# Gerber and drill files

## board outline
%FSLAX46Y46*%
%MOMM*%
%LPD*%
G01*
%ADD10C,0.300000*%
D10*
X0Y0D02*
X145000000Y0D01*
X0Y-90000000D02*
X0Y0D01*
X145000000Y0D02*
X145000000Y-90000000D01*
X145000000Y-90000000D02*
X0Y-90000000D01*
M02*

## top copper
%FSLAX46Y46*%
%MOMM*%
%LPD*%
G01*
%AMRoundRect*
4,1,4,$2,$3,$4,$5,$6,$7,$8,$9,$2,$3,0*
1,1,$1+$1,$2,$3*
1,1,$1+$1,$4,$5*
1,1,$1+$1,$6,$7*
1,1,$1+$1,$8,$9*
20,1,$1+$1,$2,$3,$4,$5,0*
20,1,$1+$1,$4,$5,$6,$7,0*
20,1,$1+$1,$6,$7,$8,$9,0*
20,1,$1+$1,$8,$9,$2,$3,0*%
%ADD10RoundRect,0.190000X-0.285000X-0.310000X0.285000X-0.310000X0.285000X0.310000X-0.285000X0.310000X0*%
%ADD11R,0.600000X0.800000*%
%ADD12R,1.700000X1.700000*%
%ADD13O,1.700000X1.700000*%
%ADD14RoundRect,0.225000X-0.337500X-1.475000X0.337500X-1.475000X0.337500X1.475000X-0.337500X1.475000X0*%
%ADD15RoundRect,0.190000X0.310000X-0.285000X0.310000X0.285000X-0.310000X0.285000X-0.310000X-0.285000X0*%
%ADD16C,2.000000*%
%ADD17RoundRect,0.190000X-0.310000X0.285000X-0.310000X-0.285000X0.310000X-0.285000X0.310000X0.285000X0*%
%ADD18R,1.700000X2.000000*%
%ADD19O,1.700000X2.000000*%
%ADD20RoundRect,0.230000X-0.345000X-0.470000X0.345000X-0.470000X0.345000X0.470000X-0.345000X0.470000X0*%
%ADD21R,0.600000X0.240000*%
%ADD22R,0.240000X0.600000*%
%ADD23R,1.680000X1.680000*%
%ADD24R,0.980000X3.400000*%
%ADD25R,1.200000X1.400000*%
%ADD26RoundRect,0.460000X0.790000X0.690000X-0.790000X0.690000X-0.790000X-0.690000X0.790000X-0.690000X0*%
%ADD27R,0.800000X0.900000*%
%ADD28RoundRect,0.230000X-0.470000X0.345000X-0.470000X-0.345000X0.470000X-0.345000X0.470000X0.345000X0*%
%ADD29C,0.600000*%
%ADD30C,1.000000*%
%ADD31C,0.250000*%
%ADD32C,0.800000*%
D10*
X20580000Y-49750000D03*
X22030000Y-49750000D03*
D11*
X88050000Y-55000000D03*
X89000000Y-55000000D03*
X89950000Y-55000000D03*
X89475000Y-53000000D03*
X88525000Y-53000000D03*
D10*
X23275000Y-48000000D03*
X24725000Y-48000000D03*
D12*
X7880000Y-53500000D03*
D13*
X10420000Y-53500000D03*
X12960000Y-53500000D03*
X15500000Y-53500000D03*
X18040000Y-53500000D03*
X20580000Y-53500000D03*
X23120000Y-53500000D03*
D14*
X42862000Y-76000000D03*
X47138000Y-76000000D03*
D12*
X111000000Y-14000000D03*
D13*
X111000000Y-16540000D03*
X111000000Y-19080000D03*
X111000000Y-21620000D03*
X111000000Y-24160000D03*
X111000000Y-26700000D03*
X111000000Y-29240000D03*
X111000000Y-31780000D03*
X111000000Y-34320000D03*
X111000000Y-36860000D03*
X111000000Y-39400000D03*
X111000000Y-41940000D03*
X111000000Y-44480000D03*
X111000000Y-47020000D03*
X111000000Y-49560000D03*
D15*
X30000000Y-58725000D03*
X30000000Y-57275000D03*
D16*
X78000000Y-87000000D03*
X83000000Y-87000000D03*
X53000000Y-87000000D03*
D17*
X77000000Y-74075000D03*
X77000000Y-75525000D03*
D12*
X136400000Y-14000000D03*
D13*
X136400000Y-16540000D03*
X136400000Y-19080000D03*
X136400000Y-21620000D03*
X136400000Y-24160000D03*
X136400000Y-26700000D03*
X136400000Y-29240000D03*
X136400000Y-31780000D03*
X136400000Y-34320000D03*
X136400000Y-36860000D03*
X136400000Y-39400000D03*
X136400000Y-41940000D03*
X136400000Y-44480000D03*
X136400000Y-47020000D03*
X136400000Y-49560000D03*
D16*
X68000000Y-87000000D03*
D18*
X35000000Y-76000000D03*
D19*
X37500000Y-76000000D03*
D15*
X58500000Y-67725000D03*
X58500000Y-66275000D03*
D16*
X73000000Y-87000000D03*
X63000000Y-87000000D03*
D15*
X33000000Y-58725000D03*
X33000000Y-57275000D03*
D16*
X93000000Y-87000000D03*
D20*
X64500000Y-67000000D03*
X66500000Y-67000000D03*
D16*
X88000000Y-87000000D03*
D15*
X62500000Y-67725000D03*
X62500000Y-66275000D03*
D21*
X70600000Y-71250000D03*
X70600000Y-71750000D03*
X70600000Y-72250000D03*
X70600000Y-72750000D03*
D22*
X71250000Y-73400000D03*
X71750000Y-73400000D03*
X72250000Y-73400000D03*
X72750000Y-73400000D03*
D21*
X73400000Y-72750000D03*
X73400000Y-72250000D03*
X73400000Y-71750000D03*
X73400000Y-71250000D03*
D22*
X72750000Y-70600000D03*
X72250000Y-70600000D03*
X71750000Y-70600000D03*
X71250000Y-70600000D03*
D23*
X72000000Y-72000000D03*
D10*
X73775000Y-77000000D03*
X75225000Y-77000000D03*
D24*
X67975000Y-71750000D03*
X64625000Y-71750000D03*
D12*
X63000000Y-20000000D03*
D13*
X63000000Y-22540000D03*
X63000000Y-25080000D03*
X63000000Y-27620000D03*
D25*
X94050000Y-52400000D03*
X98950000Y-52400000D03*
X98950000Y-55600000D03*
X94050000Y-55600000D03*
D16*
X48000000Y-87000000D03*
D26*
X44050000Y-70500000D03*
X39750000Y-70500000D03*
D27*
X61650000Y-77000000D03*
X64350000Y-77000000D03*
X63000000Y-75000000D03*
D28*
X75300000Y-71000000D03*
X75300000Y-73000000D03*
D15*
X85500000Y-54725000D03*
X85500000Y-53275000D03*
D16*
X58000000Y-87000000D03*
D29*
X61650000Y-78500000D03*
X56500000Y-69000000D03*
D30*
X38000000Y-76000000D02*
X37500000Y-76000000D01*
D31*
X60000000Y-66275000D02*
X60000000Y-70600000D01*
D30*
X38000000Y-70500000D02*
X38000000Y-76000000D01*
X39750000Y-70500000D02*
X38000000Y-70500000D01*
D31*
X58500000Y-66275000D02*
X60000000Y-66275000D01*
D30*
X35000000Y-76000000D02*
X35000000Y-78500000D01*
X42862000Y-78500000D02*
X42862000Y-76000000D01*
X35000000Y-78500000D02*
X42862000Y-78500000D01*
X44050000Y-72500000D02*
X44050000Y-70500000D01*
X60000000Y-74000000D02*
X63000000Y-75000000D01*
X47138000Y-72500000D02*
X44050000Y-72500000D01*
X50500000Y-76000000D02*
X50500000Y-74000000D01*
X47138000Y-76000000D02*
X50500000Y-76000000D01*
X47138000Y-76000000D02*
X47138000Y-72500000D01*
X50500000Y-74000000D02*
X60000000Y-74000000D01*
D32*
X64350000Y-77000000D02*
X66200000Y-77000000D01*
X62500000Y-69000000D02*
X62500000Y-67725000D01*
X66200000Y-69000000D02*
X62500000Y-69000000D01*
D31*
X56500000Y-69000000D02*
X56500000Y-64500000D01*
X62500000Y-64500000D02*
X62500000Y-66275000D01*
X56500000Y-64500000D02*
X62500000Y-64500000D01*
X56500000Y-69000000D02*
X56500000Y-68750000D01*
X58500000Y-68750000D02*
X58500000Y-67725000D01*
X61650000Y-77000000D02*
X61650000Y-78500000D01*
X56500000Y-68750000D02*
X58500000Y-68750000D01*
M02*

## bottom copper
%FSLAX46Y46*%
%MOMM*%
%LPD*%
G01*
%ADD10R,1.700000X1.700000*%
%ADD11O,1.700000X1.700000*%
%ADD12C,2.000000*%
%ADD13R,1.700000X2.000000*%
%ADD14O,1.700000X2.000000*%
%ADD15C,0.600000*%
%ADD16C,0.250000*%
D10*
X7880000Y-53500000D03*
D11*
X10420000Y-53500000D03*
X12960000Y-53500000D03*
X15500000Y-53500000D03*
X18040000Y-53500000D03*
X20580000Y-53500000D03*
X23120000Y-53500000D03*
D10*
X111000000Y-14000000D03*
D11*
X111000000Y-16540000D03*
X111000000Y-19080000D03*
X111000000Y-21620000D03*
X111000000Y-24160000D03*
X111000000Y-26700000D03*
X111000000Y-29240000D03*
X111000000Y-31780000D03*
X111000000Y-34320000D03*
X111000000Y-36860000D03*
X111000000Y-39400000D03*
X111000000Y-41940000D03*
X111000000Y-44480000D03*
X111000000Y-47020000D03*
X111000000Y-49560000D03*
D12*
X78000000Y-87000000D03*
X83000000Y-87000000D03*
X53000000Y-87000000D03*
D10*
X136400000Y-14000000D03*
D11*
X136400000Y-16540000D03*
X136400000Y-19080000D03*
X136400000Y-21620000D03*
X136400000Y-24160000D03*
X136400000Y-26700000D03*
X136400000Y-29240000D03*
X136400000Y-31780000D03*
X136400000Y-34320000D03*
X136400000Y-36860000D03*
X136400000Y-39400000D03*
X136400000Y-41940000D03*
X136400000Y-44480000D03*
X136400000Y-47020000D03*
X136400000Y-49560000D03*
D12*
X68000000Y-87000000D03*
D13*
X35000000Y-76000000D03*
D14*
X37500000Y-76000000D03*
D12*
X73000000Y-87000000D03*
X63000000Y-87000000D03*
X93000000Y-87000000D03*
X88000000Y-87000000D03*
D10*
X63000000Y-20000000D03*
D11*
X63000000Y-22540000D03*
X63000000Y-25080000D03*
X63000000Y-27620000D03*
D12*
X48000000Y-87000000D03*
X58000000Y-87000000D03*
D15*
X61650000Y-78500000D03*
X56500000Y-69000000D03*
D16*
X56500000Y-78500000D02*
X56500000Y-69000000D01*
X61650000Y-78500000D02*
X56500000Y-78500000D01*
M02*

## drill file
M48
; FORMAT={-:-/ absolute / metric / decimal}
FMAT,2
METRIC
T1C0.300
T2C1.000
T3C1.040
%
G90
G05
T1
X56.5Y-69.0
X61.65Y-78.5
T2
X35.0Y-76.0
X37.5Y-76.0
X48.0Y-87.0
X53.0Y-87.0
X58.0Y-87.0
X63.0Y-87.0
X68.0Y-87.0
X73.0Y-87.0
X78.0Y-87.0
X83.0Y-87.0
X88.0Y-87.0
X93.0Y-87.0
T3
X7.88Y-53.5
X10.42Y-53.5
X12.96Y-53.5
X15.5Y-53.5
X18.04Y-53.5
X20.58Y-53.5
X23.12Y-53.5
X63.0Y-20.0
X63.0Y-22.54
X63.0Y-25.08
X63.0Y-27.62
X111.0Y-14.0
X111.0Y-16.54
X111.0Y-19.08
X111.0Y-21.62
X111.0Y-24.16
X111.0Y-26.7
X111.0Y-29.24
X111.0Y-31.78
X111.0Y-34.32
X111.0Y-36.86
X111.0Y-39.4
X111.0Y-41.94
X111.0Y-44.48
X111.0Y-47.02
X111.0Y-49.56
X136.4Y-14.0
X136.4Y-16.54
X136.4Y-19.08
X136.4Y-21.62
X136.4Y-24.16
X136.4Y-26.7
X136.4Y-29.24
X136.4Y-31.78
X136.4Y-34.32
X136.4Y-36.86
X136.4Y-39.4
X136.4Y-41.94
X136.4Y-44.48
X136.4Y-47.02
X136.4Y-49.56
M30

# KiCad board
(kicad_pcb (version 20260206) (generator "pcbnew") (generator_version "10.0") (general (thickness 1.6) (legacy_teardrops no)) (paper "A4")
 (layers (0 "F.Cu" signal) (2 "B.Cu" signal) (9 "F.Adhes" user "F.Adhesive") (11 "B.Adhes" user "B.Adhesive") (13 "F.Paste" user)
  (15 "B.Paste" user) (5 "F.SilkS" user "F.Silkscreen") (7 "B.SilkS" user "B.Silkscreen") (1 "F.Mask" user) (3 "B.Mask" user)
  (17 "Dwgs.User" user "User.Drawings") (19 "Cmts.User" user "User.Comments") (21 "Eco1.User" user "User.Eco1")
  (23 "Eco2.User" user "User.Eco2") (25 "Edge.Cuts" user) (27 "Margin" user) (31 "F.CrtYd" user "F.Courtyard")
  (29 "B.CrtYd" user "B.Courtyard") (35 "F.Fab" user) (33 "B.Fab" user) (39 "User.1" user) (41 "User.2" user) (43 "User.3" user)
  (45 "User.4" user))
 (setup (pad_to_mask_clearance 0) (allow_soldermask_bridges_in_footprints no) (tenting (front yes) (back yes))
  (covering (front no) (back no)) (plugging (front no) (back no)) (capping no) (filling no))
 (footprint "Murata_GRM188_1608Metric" (layer "F.Cu") (at 21.305 49.75)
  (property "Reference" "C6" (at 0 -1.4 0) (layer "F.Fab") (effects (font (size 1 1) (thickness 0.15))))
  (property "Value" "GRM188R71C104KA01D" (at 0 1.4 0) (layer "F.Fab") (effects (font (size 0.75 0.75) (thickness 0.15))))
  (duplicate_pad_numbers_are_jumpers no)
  (pad "1" smd roundrect (at -0.725 0) (size 0.95 1) (layers "F.Cu" "F.Mask" "F.Paste") (roundrect_rratio 0.2) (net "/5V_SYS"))
  (pad "2" smd roundrect (at 0.725 0) (size 0.95 1) (layers "F.Cu" "F.Mask" "F.Paste") (roundrect_rratio 0.2) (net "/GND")))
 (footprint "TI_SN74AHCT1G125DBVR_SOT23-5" (layer "F.Cu") (at 89 54)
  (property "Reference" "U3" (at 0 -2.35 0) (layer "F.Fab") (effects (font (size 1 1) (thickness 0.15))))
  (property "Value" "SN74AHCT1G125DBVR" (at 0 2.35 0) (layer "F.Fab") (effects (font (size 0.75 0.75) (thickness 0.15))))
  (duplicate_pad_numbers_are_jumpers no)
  (pad "1" smd rect (at -0.95 1) (size 0.6 0.8) (layers "F.Cu" "F.Mask" "F.Paste") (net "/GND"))
  (pad "2" smd rect (at 0 1) (size 0.6 0.8) (layers "F.Cu" "F.Mask" "F.Paste") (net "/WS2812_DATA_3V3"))
  (pad "3" smd rect (at 0.95 1) (size 0.6 0.8) (layers "F.Cu" "F.Mask" "F.Paste") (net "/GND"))
  (pad "4" smd rect (at 0.475 -1) (size 0.6 0.8) (layers "F.Cu" "F.Mask" "F.Paste") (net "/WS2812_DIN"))
  (pad "5" smd rect (at -0.475 -1) (size 0.6 0.8) (layers "F.Cu" "F.Mask" "F.Paste") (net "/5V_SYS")))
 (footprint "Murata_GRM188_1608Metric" (layer "F.Cu") (at 24 48)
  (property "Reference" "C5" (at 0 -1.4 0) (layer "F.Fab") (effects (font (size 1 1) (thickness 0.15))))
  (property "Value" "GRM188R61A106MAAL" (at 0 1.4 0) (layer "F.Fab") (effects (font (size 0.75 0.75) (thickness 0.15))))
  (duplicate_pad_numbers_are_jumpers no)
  (pad "1" smd roundrect (at -0.725 0) (size 0.95 1) (layers "F.Cu" "F.Mask" "F.Paste") (roundrect_rratio 0.2) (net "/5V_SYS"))
  (pad "2" smd roundrect (at 0.725 0) (size 0.95 1) (layers "F.Cu" "F.Mask" "F.Paste") (roundrect_rratio 0.2) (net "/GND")))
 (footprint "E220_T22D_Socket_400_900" (layer "F.Cu") (at 5 52)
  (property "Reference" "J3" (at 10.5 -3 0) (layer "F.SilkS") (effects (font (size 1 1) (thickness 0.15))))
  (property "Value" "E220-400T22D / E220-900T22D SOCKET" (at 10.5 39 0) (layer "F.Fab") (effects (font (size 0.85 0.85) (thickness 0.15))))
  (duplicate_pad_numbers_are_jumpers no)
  (pad "1" thru_hole rect (at 2.88 1.5) (size 1.7 1.7) (drill 1.04) (layers "*.Cu" "*.Mask") (remove_unused_layers no) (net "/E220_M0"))
  (pad "2" thru_hole oval (at 5.42 1.5) (size 1.7 1.7) (drill 1.04) (layers "*.Cu" "*.Mask") (remove_unused_layers no) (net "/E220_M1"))
  (pad "3" thru_hole oval (at 7.96 1.5) (size 1.7 1.7) (drill 1.04) (layers "*.Cu" "*.Mask") (remove_unused_layers no) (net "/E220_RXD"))
  (pad "4" thru_hole oval (at 10.5 1.5) (size 1.7 1.7) (drill 1.04) (layers "*.Cu" "*.Mask") (remove_unused_layers no) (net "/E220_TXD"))
  (pad "5" thru_hole oval (at 13.04 1.5) (size 1.7 1.7) (drill 1.04) (layers "*.Cu" "*.Mask") (remove_unused_layers no) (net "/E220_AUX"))
  (pad "6" thru_hole oval (at 15.58 1.5) (size 1.7 1.7) (drill 1.04) (layers "*.Cu" "*.Mask") (remove_unused_layers no) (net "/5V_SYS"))
  (pad "7" thru_hole oval (at 18.12 1.5) (size 1.7 1.7) (drill 1.04) (layers "*.Cu" "*.Mask") (remove_unused_layers no) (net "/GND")))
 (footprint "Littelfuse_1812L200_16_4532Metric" (layer "F.Cu") (at 45 76)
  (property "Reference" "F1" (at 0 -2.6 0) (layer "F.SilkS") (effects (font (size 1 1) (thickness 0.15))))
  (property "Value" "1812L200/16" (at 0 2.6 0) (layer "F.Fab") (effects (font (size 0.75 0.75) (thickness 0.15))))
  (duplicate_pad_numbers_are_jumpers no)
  (pad "1" smd roundrect (at -2.138 0) (size 1.125 3.4) (layers "F.Cu" "F.Mask" "F.Paste") (roundrect_rratio 0.2) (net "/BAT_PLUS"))
  (pad "2" smd roundrect (at 2.138 0) (size 1.125 3.4) (layers "F.Cu" "F.Mask" "F.Paste") (roundrect_rratio 0.2) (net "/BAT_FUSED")))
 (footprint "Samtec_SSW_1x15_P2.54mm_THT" (layer "F.Cu") (at 111 14)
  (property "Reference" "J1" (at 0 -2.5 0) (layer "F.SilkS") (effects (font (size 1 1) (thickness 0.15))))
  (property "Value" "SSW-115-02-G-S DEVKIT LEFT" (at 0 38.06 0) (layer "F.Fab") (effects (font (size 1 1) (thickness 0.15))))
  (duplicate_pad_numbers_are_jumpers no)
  (pad "1" thru_hole rect (at 0 0) (size 1.7 1.7) (drill 1.04) (layers "*.Cu" "*.Mask") (remove_unused_layers no) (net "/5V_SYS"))
  (pad "2" thru_hole oval (at 0 2.54) (size 1.7 1.7) (drill 1.04) (layers "*.Cu" "*.Mask") (remove_unused_layers no) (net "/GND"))
  (pad "3" thru_hole oval (at 0 5.08) (size 1.7 1.7) (drill 1.04) (layers "*.Cu" "*.Mask") (remove_unused_layers no))
  (pad "4" thru_hole oval (at 0 7.62) (size 1.7 1.7) (drill 1.04) (layers "*.Cu" "*.Mask") (remove_unused_layers no))
  (pad "5" thru_hole oval (at 0 10.16) (size 1.7 1.7) (drill 1.04) (layers "*.Cu" "*.Mask") (remove_unused_layers no))
  (pad "6" thru_hole oval (at 0 12.7) (size 1.7 1.7) (drill 1.04) (layers "*.Cu" "*.Mask") (remove_unused_layers no) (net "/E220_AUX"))
  (pad "7" thru_hole oval (at 0 15.24) (size 1.7 1.7) (drill 1.04) (layers "*.Cu" "*.Mask") (remove_unused_layers no) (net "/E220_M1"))
  (pad "8" thru_hole oval (at 0 17.78) (size 1.7 1.7) (drill 1.04) (layers "*.Cu" "*.Mask") (remove_unused_layers no) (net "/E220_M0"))
  (pad "9" thru_hole oval (at 0 20.32) (size 1.7 1.7) (drill 1.04) (layers "*.Cu" "*.Mask") (remove_unused_layers no))
  (pad "10" thru_hole oval (at 0 22.86) (size 1.7 1.7) (drill 1.04) (layers "*.Cu" "*.Mask") (remove_unused_layers no))
  (pad "11" thru_hole oval (at 0 25.4) (size 1.7 1.7) (drill 1.04) (layers "*.Cu" "*.Mask") (remove_unused_layers no))
  (pad "12" thru_hole oval (at 0 27.94) (size 1.7 1.7) (drill 1.04) (layers "*.Cu" "*.Mask") (remove_unused_layers no))
  (pad "13" thru_hole oval (at 0 30.48) (size 1.7 1.7) (drill 1.04) (layers "*.Cu" "*.Mask") (remove_unused_layers no))
  (pad "14" thru_hole oval (at 0 33.02) (size 1.7 1.7) (drill 1.04) (layers "*.Cu" "*.Mask") (remove_unused_layers no))
  (pad "15" thru_hole oval (at 0 35.56) (size 1.7 1.7) (drill 1.04) (layers "*.Cu" "*.Mask") (remove_unused_layers no)))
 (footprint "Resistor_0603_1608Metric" (layer "F.Cu") (at 30 58 90)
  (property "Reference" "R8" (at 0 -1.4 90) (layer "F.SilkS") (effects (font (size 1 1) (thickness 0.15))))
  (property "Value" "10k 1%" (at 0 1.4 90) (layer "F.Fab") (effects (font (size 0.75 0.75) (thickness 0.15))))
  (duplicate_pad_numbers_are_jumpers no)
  (pad "1" smd roundrect (at -0.725 0 90) (size 0.95 1) (layers "F.Cu" "F.Mask" "F.Paste") (roundrect_rratio 0.2) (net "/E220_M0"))
  (pad "2" smd roundrect (at 0.725 0 90) (size 0.95 1) (layers "F.Cu" "F.Mask" "F.Paste") (roundrect_rratio 0.2) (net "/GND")))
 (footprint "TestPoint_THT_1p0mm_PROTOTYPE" (layer "F.Cu") (at 78 87)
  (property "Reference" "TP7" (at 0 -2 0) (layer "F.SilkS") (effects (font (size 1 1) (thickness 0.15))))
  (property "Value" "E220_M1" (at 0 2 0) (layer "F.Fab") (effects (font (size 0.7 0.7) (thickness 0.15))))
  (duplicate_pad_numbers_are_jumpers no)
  (pad "1" thru_hole circle (at 0 0) (size 2 2) (drill 1) (layers "*.Cu" "*.Mask") (remove_unused_layers no) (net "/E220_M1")))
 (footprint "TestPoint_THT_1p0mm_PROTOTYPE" (layer "F.Cu") (at 83 87)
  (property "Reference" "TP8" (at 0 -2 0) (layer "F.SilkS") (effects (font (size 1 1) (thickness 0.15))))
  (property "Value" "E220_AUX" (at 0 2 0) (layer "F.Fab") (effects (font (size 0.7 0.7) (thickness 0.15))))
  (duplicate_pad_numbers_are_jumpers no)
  (pad "1" thru_hole circle (at 0 0) (size 2 2) (drill 1) (layers "*.Cu" "*.Mask") (remove_unused_layers no) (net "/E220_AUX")))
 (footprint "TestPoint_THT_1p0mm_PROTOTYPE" (layer "F.Cu") (at 53 87)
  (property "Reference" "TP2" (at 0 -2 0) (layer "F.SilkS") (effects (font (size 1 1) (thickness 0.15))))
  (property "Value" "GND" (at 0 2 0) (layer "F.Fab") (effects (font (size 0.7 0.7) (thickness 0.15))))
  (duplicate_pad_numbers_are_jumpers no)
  (pad "1" thru_hole circle (at 0 0) (size 2 2) (drill 1) (layers "*.Cu" "*.Mask") (remove_unused_layers no) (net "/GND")))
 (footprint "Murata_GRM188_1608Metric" (layer "F.Cu") (at 77 74.8 -90)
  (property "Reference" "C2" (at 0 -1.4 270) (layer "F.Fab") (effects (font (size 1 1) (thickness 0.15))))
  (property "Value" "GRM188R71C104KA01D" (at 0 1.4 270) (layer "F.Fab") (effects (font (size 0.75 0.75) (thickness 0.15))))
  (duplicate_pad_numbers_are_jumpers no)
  (pad "1" smd roundrect (at -0.725 0 270) (size 0.95 1) (layers "F.Cu" "F.Mask" "F.Paste") (roundrect_rratio 0.2) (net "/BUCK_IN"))
  (pad "2" smd roundrect (at 0.725 0 270) (size 0.95 1) (layers "F.Cu" "F.Mask" "F.Paste") (roundrect_rratio 0.2) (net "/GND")))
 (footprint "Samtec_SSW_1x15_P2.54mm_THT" (layer "F.Cu") (at 136.4 14)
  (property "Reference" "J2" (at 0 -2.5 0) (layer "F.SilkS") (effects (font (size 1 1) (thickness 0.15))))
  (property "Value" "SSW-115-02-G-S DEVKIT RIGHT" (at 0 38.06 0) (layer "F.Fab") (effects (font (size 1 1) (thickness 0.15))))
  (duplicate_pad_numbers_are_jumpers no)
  (pad "1" thru_hole rect (at 0 0) (size 1.7 1.7) (drill 1.04) (layers "*.Cu" "*.Mask") (remove_unused_layers no) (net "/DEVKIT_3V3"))
  (pad "2" thru_hole oval (at 0 2.54) (size 1.7 1.7) (drill 1.04) (layers "*.Cu" "*.Mask") (remove_unused_layers no) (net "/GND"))
  (pad "3" thru_hole oval (at 0 5.08) (size 1.7 1.7) (drill 1.04) (layers "*.Cu" "*.Mask") (remove_unused_layers no))
  (pad "4" thru_hole oval (at 0 7.62) (size 1.7 1.7) (drill 1.04) (layers "*.Cu" "*.Mask") (remove_unused_layers no))
  (pad "5" thru_hole oval (at 0 10.16) (size 1.7 1.7) (drill 1.04) (layers "*.Cu" "*.Mask") (remove_unused_layers no)
   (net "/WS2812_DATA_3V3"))
  (pad "6" thru_hole oval (at 0 12.7) (size 1.7 1.7) (drill 1.04) (layers "*.Cu" "*.Mask") (remove_unused_layers no) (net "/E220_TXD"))
  (pad "7" thru_hole oval (at 0 15.24) (size 1.7 1.7) (drill 1.04) (layers "*.Cu" "*.Mask") (remove_unused_layers no) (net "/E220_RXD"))
  (pad "8" thru_hole oval (at 0 17.78) (size 1.7 1.7) (drill 1.04) (layers "*.Cu" "*.Mask") (remove_unused_layers no))
  (pad "9" thru_hole oval (at 0 20.32) (size 1.7 1.7) (drill 1.04) (layers "*.Cu" "*.Mask") (remove_unused_layers no))
  (pad "10" thru_hole oval (at 0 22.86) (size 1.7 1.7) (drill 1.04) (layers "*.Cu" "*.Mask") (remove_unused_layers no))
  (pad "11" thru_hole oval (at 0 25.4) (size 1.7 1.7) (drill 1.04) (layers "*.Cu" "*.Mask") (remove_unused_layers no) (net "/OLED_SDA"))
  (pad "12" thru_hole oval (at 0 27.94) (size 1.7 1.7) (drill 1.04) (layers "*.Cu" "*.Mask") (remove_unused_layers no))
  (pad "13" thru_hole oval (at 0 30.48) (size 1.7 1.7) (drill 1.04) (layers "*.Cu" "*.Mask") (remove_unused_layers no))
  (pad "14" thru_hole oval (at 0 33.02) (size 1.7 1.7) (drill 1.04) (layers "*.Cu" "*.Mask") (remove_unused_layers no) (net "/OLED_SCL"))
  (pad "15" thru_hole oval (at 0 35.56) (size 1.7 1.7) (drill 1.04) (layers "*.Cu" "*.Mask") (remove_unused_layers no)))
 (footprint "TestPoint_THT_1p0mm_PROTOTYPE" (layer "F.Cu") (at 68 87)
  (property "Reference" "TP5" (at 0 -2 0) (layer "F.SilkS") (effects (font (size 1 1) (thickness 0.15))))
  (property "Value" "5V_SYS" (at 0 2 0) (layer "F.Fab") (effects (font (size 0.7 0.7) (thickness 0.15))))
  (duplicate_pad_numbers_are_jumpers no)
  (pad "1" thru_hole circle (at 0 0) (size 2 2) (drill 1) (layers "*.Cu" "*.Mask") (remove_unused_layers no) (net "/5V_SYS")))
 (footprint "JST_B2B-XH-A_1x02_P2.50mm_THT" (layer "F.Cu") (at 35 76)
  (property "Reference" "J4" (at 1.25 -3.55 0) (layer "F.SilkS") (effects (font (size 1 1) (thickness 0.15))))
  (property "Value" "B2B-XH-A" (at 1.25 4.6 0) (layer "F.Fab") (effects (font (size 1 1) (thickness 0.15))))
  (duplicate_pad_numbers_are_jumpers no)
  (pad "1" thru_hole rect (at 0 0) (size 1.7 2) (drill 1) (layers "*.Cu" "*.Mask") (remove_unused_layers no) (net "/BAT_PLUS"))
  (pad "2" thru_hole oval (at 2.5 0) (size 1.7 2) (drill 1) (layers "*.Cu" "*.Mask") (remove_unused_layers no) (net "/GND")))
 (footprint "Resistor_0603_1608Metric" (layer "F.Cu") (at 58.5 67 90)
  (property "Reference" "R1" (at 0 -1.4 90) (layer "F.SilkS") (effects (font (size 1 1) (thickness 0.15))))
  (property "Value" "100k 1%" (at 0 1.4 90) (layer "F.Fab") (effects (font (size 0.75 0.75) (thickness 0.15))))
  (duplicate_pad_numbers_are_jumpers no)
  (pad "1" smd roundrect (at -0.725 0 90) (size 0.95 1) (layers "F.Cu" "F.Mask" "F.Paste") (roundrect_rratio 0.2) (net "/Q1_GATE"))
  (pad "2" smd roundrect (at 0.725 0 90) (size 0.95 1) (layers "F.Cu" "F.Mask" "F.Paste") (roundrect_rratio 0.2) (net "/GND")))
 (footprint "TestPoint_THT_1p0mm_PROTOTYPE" (layer "F.Cu") (at 73 87)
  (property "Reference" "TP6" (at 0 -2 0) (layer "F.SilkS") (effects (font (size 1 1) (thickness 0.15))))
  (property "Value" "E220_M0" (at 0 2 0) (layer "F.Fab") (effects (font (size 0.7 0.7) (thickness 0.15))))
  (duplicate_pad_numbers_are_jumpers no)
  (pad "1" thru_hole circle (at 0 0) (size 2 2) (drill 1) (layers "*.Cu" "*.Mask") (remove_unused_layers no) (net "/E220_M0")))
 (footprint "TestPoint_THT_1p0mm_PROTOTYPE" (layer "F.Cu") (at 63 87)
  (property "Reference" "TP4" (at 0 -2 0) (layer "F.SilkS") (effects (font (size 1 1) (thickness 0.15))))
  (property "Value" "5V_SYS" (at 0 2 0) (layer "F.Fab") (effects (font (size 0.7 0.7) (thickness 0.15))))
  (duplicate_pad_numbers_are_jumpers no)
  (pad "1" thru_hole circle (at 0 0) (size 2 2) (drill 1) (layers "*.Cu" "*.Mask") (remove_unused_layers no) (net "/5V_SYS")))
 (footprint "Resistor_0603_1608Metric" (layer "F.Cu") (at 33 58 90)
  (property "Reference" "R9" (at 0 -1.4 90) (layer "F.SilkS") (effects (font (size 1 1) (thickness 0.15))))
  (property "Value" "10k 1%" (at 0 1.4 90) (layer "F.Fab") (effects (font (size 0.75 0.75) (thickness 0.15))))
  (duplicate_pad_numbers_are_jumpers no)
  (pad "1" smd roundrect (at -0.725 0 90) (size 0.95 1) (layers "F.Cu" "F.Mask" "F.Paste") (roundrect_rratio 0.2) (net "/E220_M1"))
  (pad "2" smd roundrect (at 0.725 0 90) (size 0.95 1) (layers "F.Cu" "F.Mask" "F.Paste") (roundrect_rratio 0.2) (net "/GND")))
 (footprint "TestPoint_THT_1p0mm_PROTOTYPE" (layer "F.Cu") (at 93 87)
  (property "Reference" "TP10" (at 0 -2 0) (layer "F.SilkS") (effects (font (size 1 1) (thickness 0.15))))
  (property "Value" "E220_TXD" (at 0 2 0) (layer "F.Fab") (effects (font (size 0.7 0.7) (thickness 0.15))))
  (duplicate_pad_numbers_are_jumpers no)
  (pad "1" thru_hole circle (at 0 0) (size 2 2) (drill 1) (layers "*.Cu" "*.Mask") (remove_unused_layers no) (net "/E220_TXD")))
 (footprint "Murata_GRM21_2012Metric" (layer "F.Cu") (at 65.5 67)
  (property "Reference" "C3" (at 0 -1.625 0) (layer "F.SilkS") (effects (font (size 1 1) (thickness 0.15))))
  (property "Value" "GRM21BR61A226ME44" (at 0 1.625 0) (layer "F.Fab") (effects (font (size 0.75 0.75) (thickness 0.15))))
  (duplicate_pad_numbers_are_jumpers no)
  (pad "1" smd roundrect (at -1 0) (size 1.15 1.4) (layers "F.Cu" "F.Mask" "F.Paste") (roundrect_rratio 0.2) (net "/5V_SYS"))
  (pad "2" smd roundrect (at 1 0) (size 1.15 1.4) (layers "F.Cu" "F.Mask" "F.Paste") (roundrect_rratio 0.2) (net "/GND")))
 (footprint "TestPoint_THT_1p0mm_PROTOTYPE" (layer "F.Cu") (at 88 87)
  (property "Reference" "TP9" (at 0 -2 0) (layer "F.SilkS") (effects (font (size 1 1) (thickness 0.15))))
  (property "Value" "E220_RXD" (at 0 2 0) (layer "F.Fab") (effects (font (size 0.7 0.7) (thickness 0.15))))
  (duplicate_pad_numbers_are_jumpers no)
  (pad "1" thru_hole circle (at 0 0) (size 2 2) (drill 1) (layers "*.Cu" "*.Mask") (remove_unused_layers no) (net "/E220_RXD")))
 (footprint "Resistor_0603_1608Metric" (layer "F.Cu") (at 62.5 67 90)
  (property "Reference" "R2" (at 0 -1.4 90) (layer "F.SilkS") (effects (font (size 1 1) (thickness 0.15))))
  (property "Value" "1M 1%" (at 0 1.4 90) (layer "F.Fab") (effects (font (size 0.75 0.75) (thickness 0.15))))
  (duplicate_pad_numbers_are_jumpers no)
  (pad "1" smd roundrect (at -0.725 0 90) (size 0.95 1) (layers "F.Cu" "F.Mask" "F.Paste") (roundrect_rratio 0.2) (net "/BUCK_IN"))
  (pad "2" smd roundrect (at 0.725 0 90) (size 0.95 1) (layers "F.Cu" "F.Mask" "F.Paste") (roundrect_rratio 0.2) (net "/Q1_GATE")))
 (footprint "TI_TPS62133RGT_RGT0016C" (layer "F.Cu") (at 72 72)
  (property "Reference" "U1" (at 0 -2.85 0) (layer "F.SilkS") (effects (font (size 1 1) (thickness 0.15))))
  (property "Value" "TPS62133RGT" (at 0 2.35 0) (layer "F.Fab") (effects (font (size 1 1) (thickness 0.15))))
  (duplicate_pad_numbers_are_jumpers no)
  (pad "" smd rect (at 0 0) (size 1.55 1.55) (layers "F.Paste"))
  (pad "1" smd rect (at -1.4 -0.75) (size 0.6 0.24) (layers "F.Cu" "F.Mask" "F.Paste") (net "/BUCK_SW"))
  (pad "2" smd rect (at -1.4 -0.25) (size 0.6 0.24) (layers "F.Cu" "F.Mask" "F.Paste") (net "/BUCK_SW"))
  (pad "3" smd rect (at -1.4 0.25) (size 0.6 0.24) (layers "F.Cu" "F.Mask" "F.Paste") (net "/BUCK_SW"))
  (pad "4" smd rect (at -1.4 0.75) (size 0.6 0.24) (layers "F.Cu" "F.Mask" "F.Paste"))
  (pad "5" smd rect (at -0.75 1.4) (size 0.24 0.6) (layers "F.Cu" "F.Mask" "F.Paste") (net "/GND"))
  (pad "6" smd rect (at -0.25 1.4) (size 0.24 0.6) (layers "F.Cu" "F.Mask" "F.Paste") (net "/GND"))
  (pad "7" smd rect (at 0.25 1.4) (size 0.24 0.6) (layers "F.Cu" "F.Mask" "F.Paste") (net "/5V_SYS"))
  (pad "8" smd rect (at 0.75 1.4) (size 0.24 0.6) (layers "F.Cu" "F.Mask" "F.Paste") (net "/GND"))
  (pad "9" smd rect (at 1.4 0.75) (size 0.6 0.24) (layers "F.Cu" "F.Mask" "F.Paste") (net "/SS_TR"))
  (pad "10" smd rect (at 1.4 0.25) (size 0.6 0.24) (layers "F.Cu" "F.Mask" "F.Paste") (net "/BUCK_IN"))
  (pad "11" smd rect (at 1.4 -0.25) (size 0.6 0.24) (layers "F.Cu" "F.Mask" "F.Paste") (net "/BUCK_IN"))
  (pad "12" smd rect (at 1.4 -0.75) (size 0.6 0.24) (layers "F.Cu" "F.Mask" "F.Paste") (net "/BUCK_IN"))
  (pad "13" smd rect (at 0.75 -1.4) (size 0.24 0.6) (layers "F.Cu" "F.Mask" "F.Paste") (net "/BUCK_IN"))
  (pad "14" smd rect (at 0.25 -1.4) (size 0.24 0.6) (layers "F.Cu" "F.Mask" "F.Paste") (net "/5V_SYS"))
  (pad "15" smd rect (at -0.25 -1.4) (size 0.24 0.6) (layers "F.Cu" "F.Mask" "F.Paste") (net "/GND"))
  (pad "16" smd rect (at -0.75 -1.4) (size 0.24 0.6) (layers "F.Cu" "F.Mask" "F.Paste") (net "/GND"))
  (pad "EP" smd rect (at 0 0) (size 1.68 1.68) (layers "F.Cu" "F.Mask") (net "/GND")))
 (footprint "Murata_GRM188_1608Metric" (layer "F.Cu") (at 74.5 77)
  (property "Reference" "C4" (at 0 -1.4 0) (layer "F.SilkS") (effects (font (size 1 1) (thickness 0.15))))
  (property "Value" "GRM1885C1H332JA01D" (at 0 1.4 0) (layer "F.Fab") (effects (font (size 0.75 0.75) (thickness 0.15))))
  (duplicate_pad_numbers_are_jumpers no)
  (pad "1" smd roundrect (at -0.725 0) (size 0.95 1) (layers "F.Cu" "F.Mask" "F.Paste") (roundrect_rratio 0.2) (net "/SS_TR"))
  (pad "2" smd roundrect (at 0.725 0) (size 0.95 1) (layers "F.Cu" "F.Mask" "F.Paste") (roundrect_rratio 0.2) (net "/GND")))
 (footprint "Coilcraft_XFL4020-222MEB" (layer "F.Cu") (at 66.3 71.75 180)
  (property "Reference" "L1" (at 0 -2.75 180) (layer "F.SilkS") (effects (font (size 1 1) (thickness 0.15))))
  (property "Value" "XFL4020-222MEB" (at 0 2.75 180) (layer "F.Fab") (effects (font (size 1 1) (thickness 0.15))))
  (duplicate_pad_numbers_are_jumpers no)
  (pad "1" smd rect (at -1.675 0 180) (size 0.98 3.4) (layers "F.Cu" "F.Mask" "F.Paste") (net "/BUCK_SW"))
  (pad "2" smd rect (at 1.675 0 180) (size 0.98 3.4) (layers "F.Cu" "F.Mask" "F.Paste") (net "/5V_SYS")))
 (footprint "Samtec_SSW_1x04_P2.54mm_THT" (layer "F.Cu") (at 63 20)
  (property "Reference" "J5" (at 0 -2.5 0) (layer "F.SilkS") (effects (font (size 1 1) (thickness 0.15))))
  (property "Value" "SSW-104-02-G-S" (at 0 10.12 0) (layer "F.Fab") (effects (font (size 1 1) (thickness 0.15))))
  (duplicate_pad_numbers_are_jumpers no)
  (pad "1" thru_hole rect (at 0 0) (size 1.7 1.7) (drill 1.04) (layers "*.Cu" "*.Mask") (remove_unused_layers no) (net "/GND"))
  (pad "2" thru_hole oval (at 0 2.54) (size 1.7 1.7) (drill 1.04) (layers "*.Cu" "*.Mask") (remove_unused_layers no) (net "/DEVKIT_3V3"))
  (pad "3" thru_hole oval (at 0 5.08) (size 1.7 1.7) (drill 1.04) (layers "*.Cu" "*.Mask") (remove_unused_layers no) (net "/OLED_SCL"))
  (pad "4" thru_hole oval (at 0 7.62) (size 1.7 1.7) (drill 1.04) (layers "*.Cu" "*.Mask") (remove_unused_layers no) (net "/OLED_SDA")))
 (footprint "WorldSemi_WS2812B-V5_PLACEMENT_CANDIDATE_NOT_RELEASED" (layer "F.Cu") (at 96.5 54)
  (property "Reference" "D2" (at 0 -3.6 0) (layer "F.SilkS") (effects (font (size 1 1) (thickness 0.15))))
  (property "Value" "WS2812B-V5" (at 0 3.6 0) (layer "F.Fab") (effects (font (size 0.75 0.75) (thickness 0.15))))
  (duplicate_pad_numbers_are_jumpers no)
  (pad "1" smd rect (at -2.45 -1.6) (size 1.2 1.4) (layers "F.Cu" "F.Mask" "F.Paste") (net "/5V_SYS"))
  (pad "2" smd rect (at 2.45 -1.6) (size 1.2 1.4) (layers "F.Cu" "F.Mask" "F.Paste"))
  (pad "3" smd rect (at 2.45 1.6) (size 1.2 1.4) (layers "F.Cu" "F.Mask" "F.Paste") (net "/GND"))
  (pad "4" smd rect (at -2.45 1.6) (size 1.2 1.4) (layers "F.Cu" "F.Mask" "F.Paste") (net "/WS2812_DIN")))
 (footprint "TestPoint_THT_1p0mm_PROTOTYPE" (layer "F.Cu") (at 48 87)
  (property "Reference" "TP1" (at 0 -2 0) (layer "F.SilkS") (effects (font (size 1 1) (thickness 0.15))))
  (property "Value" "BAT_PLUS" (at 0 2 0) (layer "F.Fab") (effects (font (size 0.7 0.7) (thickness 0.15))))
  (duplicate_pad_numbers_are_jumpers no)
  (pad "1" thru_hole circle (at 0 0) (size 2 2) (drill 1) (layers "*.Cu" "*.Mask") (remove_unused_layers no) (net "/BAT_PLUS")))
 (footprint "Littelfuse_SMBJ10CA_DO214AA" (layer "F.Cu") (at 41.9 70.5 180)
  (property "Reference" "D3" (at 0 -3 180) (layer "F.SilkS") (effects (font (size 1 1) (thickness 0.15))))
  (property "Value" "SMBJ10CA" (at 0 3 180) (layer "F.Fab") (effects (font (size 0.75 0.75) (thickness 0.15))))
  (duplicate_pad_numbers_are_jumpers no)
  (pad "1" smd roundrect (at -2.15 0 180) (size 2.5 2.3) (layers "F.Cu" "F.Mask" "F.Paste") (roundrect_rratio 0.2) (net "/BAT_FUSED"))
  (pad "2" smd roundrect (at 2.15 0 180) (size 2.5 2.3) (layers "F.Cu" "F.Mask" "F.Paste") (roundrect_rratio 0.2) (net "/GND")))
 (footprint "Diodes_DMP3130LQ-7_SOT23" (layer "F.Cu") (at 63 76)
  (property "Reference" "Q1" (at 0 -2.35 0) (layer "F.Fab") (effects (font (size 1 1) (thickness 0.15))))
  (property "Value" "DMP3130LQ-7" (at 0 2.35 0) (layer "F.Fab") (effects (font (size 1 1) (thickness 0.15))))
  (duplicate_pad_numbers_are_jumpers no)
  (pad "1" smd rect (at -1.35 1) (size 0.8 0.9) (layers "F.Cu" "F.Mask" "F.Paste") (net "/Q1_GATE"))
  (pad "2" smd rect (at 1.35 1) (size 0.8 0.9) (layers "F.Cu" "F.Mask" "F.Paste") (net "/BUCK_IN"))
  (pad "3" smd rect (at 0 -1) (size 0.8 0.9) (layers "F.Cu" "F.Mask" "F.Paste") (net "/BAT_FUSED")))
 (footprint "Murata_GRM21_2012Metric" (layer "F.Cu") (at 75.3 72 -90)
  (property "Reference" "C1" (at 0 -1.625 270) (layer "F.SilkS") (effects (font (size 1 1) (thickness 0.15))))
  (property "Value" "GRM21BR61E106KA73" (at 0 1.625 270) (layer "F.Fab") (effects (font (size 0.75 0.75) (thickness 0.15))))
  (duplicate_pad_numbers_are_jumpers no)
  (pad "1" smd roundrect (at -1 0 270) (size 1.15 1.4) (layers "F.Cu" "F.Mask" "F.Paste") (roundrect_rratio 0.2) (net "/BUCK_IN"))
  (pad "2" smd roundrect (at 1 0 270) (size 1.15 1.4) (layers "F.Cu" "F.Mask" "F.Paste") (roundrect_rratio 0.2) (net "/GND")))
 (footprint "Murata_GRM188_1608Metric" (layer "F.Cu") (at 85.5 54 90)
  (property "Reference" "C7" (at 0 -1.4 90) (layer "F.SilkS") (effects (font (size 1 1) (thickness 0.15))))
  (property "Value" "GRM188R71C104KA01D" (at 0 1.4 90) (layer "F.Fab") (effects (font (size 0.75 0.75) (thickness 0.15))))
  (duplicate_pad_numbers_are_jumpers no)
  (pad "1" smd roundrect (at -0.725 0 90) (size 0.95 1) (layers "F.Cu" "F.Mask" "F.Paste") (roundrect_rratio 0.2) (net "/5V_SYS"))
  (pad "2" smd roundrect (at 0.725 0 90) (size 0.95 1) (layers "F.Cu" "F.Mask" "F.Paste") (roundrect_rratio 0.2) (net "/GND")))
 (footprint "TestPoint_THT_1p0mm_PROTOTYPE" (layer "F.Cu") (at 58 87)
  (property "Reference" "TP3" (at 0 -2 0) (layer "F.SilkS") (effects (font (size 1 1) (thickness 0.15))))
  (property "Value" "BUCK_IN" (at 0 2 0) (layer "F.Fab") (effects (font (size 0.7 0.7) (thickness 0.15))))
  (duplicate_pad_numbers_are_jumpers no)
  (pad "1" thru_hole circle (at 0 0) (size 2 2) (drill 1) (layers "*.Cu" "*.Mask") (remove_unused_layers no) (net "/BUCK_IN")))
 (gr_line (start 0 0) (end 145 0) (stroke (width 0.3) (type default)) (layer "Edge.Cuts"))
 (gr_line (start 0 90) (end 0 0) (stroke (width 0.3) (type default)) (layer "Edge.Cuts"))
 (gr_line (start 145 0) (end 145 90) (stroke (width 0.3) (type default)) (layer "Edge.Cuts"))
 (gr_line (start 145 90) (end 0 90) (stroke (width 0.3) (type default)) (layer "Edge.Cuts"))
 (segment (start 38 76) (end 37.5 76) (width 1) (layer "F.Cu") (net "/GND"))
 (segment (start 60 66.275) (end 60 70.6) (width 0.25) (layer "F.Cu") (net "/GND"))
 (segment (start 38 70.5) (end 38 76) (width 1) (layer "F.Cu") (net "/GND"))
 (segment (start 39.75 70.5) (end 38 70.5) (width 1) (layer "F.Cu") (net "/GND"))
 (segment (start 58.5 66.275) (end 60 66.275) (width 0.25) (layer "F.Cu") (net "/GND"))
 (segment (start 35 76) (end 35 78.5) (width 1) (layer "F.Cu") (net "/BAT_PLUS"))
 (segment (start 42.862 78.5) (end 42.862 76) (width 1) (layer "F.Cu") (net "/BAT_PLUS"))
 (segment (start 35 78.5) (end 42.862 78.5) (width 1) (layer "F.Cu") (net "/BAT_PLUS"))
 (segment (start 44.05 72.5) (end 44.05 70.5) (width 1) (layer "F.Cu") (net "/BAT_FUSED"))
 (segment (start 60 74) (end 63 75) (width 1) (layer "F.Cu") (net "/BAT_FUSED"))
 (segment (start 47.138 72.5) (end 44.05 72.5) (width 1) (layer "F.Cu") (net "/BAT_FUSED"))
 (segment (start 50.5 76) (end 50.5 74) (width 1) (layer "F.Cu") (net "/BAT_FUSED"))
 (segment (start 47.138 76) (end 50.5 76) (width 1) (layer "F.Cu") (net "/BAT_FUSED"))
 (segment (start 47.138 76) (end 47.138 72.5) (width 1) (layer "F.Cu") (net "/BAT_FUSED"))
 (segment (start 50.5 74) (end 60 74) (width 1) (layer "F.Cu") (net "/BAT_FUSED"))
 (segment (start 64.35 77) (end 66.2 77) (width 0.8) (layer "F.Cu") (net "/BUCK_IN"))
 (segment (start 62.5 69) (end 62.5 67.725) (width 0.8) (layer "F.Cu") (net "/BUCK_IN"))
 (segment (start 66.2 69) (end 62.5 69) (width 0.8) (layer "F.Cu") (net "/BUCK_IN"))
 (segment (start 56.5 69) (end 56.5 64.5) (width 0.25) (layer "F.Cu") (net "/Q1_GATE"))
 (segment (start 62.5 64.5) (end 62.5 66.275) (width 0.25) (layer "F.Cu") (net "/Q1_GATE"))
 (segment (start 56.5 64.5) (end 62.5 64.5) (width 0.25) (layer "F.Cu") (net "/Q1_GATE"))
 (segment (start 56.5 69) (end 56.5 68.75) (width 0.25) (layer "F.Cu") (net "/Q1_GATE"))
 (segment (start 58.5 68.75) (end 58.5 67.725) (width 0.25) (layer "F.Cu") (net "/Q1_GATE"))
 (segment (start 61.65 77) (end 61.65 78.5) (width 0.25) (layer "F.Cu") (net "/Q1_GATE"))
 (segment (start 56.5 68.75) (end 58.5 68.75) (width 0.25) (layer "F.Cu") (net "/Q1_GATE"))
 (via (at 61.65 78.5) (size 0.6) (drill 0.3) (layers "F.Cu" "B.Cu") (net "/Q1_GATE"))
 (via (at 56.5 69) (size 0.6) (drill 0.3) (layers "F.Cu" "B.Cu") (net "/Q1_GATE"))
 (segment (start 56.5 78.5) (end 56.5 69) (width 0.25) (layer "B.Cu") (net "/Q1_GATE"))
 (segment (start 61.65 78.5) (end 56.5 78.5) (width 0.25) (layer "B.Cu") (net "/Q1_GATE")))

